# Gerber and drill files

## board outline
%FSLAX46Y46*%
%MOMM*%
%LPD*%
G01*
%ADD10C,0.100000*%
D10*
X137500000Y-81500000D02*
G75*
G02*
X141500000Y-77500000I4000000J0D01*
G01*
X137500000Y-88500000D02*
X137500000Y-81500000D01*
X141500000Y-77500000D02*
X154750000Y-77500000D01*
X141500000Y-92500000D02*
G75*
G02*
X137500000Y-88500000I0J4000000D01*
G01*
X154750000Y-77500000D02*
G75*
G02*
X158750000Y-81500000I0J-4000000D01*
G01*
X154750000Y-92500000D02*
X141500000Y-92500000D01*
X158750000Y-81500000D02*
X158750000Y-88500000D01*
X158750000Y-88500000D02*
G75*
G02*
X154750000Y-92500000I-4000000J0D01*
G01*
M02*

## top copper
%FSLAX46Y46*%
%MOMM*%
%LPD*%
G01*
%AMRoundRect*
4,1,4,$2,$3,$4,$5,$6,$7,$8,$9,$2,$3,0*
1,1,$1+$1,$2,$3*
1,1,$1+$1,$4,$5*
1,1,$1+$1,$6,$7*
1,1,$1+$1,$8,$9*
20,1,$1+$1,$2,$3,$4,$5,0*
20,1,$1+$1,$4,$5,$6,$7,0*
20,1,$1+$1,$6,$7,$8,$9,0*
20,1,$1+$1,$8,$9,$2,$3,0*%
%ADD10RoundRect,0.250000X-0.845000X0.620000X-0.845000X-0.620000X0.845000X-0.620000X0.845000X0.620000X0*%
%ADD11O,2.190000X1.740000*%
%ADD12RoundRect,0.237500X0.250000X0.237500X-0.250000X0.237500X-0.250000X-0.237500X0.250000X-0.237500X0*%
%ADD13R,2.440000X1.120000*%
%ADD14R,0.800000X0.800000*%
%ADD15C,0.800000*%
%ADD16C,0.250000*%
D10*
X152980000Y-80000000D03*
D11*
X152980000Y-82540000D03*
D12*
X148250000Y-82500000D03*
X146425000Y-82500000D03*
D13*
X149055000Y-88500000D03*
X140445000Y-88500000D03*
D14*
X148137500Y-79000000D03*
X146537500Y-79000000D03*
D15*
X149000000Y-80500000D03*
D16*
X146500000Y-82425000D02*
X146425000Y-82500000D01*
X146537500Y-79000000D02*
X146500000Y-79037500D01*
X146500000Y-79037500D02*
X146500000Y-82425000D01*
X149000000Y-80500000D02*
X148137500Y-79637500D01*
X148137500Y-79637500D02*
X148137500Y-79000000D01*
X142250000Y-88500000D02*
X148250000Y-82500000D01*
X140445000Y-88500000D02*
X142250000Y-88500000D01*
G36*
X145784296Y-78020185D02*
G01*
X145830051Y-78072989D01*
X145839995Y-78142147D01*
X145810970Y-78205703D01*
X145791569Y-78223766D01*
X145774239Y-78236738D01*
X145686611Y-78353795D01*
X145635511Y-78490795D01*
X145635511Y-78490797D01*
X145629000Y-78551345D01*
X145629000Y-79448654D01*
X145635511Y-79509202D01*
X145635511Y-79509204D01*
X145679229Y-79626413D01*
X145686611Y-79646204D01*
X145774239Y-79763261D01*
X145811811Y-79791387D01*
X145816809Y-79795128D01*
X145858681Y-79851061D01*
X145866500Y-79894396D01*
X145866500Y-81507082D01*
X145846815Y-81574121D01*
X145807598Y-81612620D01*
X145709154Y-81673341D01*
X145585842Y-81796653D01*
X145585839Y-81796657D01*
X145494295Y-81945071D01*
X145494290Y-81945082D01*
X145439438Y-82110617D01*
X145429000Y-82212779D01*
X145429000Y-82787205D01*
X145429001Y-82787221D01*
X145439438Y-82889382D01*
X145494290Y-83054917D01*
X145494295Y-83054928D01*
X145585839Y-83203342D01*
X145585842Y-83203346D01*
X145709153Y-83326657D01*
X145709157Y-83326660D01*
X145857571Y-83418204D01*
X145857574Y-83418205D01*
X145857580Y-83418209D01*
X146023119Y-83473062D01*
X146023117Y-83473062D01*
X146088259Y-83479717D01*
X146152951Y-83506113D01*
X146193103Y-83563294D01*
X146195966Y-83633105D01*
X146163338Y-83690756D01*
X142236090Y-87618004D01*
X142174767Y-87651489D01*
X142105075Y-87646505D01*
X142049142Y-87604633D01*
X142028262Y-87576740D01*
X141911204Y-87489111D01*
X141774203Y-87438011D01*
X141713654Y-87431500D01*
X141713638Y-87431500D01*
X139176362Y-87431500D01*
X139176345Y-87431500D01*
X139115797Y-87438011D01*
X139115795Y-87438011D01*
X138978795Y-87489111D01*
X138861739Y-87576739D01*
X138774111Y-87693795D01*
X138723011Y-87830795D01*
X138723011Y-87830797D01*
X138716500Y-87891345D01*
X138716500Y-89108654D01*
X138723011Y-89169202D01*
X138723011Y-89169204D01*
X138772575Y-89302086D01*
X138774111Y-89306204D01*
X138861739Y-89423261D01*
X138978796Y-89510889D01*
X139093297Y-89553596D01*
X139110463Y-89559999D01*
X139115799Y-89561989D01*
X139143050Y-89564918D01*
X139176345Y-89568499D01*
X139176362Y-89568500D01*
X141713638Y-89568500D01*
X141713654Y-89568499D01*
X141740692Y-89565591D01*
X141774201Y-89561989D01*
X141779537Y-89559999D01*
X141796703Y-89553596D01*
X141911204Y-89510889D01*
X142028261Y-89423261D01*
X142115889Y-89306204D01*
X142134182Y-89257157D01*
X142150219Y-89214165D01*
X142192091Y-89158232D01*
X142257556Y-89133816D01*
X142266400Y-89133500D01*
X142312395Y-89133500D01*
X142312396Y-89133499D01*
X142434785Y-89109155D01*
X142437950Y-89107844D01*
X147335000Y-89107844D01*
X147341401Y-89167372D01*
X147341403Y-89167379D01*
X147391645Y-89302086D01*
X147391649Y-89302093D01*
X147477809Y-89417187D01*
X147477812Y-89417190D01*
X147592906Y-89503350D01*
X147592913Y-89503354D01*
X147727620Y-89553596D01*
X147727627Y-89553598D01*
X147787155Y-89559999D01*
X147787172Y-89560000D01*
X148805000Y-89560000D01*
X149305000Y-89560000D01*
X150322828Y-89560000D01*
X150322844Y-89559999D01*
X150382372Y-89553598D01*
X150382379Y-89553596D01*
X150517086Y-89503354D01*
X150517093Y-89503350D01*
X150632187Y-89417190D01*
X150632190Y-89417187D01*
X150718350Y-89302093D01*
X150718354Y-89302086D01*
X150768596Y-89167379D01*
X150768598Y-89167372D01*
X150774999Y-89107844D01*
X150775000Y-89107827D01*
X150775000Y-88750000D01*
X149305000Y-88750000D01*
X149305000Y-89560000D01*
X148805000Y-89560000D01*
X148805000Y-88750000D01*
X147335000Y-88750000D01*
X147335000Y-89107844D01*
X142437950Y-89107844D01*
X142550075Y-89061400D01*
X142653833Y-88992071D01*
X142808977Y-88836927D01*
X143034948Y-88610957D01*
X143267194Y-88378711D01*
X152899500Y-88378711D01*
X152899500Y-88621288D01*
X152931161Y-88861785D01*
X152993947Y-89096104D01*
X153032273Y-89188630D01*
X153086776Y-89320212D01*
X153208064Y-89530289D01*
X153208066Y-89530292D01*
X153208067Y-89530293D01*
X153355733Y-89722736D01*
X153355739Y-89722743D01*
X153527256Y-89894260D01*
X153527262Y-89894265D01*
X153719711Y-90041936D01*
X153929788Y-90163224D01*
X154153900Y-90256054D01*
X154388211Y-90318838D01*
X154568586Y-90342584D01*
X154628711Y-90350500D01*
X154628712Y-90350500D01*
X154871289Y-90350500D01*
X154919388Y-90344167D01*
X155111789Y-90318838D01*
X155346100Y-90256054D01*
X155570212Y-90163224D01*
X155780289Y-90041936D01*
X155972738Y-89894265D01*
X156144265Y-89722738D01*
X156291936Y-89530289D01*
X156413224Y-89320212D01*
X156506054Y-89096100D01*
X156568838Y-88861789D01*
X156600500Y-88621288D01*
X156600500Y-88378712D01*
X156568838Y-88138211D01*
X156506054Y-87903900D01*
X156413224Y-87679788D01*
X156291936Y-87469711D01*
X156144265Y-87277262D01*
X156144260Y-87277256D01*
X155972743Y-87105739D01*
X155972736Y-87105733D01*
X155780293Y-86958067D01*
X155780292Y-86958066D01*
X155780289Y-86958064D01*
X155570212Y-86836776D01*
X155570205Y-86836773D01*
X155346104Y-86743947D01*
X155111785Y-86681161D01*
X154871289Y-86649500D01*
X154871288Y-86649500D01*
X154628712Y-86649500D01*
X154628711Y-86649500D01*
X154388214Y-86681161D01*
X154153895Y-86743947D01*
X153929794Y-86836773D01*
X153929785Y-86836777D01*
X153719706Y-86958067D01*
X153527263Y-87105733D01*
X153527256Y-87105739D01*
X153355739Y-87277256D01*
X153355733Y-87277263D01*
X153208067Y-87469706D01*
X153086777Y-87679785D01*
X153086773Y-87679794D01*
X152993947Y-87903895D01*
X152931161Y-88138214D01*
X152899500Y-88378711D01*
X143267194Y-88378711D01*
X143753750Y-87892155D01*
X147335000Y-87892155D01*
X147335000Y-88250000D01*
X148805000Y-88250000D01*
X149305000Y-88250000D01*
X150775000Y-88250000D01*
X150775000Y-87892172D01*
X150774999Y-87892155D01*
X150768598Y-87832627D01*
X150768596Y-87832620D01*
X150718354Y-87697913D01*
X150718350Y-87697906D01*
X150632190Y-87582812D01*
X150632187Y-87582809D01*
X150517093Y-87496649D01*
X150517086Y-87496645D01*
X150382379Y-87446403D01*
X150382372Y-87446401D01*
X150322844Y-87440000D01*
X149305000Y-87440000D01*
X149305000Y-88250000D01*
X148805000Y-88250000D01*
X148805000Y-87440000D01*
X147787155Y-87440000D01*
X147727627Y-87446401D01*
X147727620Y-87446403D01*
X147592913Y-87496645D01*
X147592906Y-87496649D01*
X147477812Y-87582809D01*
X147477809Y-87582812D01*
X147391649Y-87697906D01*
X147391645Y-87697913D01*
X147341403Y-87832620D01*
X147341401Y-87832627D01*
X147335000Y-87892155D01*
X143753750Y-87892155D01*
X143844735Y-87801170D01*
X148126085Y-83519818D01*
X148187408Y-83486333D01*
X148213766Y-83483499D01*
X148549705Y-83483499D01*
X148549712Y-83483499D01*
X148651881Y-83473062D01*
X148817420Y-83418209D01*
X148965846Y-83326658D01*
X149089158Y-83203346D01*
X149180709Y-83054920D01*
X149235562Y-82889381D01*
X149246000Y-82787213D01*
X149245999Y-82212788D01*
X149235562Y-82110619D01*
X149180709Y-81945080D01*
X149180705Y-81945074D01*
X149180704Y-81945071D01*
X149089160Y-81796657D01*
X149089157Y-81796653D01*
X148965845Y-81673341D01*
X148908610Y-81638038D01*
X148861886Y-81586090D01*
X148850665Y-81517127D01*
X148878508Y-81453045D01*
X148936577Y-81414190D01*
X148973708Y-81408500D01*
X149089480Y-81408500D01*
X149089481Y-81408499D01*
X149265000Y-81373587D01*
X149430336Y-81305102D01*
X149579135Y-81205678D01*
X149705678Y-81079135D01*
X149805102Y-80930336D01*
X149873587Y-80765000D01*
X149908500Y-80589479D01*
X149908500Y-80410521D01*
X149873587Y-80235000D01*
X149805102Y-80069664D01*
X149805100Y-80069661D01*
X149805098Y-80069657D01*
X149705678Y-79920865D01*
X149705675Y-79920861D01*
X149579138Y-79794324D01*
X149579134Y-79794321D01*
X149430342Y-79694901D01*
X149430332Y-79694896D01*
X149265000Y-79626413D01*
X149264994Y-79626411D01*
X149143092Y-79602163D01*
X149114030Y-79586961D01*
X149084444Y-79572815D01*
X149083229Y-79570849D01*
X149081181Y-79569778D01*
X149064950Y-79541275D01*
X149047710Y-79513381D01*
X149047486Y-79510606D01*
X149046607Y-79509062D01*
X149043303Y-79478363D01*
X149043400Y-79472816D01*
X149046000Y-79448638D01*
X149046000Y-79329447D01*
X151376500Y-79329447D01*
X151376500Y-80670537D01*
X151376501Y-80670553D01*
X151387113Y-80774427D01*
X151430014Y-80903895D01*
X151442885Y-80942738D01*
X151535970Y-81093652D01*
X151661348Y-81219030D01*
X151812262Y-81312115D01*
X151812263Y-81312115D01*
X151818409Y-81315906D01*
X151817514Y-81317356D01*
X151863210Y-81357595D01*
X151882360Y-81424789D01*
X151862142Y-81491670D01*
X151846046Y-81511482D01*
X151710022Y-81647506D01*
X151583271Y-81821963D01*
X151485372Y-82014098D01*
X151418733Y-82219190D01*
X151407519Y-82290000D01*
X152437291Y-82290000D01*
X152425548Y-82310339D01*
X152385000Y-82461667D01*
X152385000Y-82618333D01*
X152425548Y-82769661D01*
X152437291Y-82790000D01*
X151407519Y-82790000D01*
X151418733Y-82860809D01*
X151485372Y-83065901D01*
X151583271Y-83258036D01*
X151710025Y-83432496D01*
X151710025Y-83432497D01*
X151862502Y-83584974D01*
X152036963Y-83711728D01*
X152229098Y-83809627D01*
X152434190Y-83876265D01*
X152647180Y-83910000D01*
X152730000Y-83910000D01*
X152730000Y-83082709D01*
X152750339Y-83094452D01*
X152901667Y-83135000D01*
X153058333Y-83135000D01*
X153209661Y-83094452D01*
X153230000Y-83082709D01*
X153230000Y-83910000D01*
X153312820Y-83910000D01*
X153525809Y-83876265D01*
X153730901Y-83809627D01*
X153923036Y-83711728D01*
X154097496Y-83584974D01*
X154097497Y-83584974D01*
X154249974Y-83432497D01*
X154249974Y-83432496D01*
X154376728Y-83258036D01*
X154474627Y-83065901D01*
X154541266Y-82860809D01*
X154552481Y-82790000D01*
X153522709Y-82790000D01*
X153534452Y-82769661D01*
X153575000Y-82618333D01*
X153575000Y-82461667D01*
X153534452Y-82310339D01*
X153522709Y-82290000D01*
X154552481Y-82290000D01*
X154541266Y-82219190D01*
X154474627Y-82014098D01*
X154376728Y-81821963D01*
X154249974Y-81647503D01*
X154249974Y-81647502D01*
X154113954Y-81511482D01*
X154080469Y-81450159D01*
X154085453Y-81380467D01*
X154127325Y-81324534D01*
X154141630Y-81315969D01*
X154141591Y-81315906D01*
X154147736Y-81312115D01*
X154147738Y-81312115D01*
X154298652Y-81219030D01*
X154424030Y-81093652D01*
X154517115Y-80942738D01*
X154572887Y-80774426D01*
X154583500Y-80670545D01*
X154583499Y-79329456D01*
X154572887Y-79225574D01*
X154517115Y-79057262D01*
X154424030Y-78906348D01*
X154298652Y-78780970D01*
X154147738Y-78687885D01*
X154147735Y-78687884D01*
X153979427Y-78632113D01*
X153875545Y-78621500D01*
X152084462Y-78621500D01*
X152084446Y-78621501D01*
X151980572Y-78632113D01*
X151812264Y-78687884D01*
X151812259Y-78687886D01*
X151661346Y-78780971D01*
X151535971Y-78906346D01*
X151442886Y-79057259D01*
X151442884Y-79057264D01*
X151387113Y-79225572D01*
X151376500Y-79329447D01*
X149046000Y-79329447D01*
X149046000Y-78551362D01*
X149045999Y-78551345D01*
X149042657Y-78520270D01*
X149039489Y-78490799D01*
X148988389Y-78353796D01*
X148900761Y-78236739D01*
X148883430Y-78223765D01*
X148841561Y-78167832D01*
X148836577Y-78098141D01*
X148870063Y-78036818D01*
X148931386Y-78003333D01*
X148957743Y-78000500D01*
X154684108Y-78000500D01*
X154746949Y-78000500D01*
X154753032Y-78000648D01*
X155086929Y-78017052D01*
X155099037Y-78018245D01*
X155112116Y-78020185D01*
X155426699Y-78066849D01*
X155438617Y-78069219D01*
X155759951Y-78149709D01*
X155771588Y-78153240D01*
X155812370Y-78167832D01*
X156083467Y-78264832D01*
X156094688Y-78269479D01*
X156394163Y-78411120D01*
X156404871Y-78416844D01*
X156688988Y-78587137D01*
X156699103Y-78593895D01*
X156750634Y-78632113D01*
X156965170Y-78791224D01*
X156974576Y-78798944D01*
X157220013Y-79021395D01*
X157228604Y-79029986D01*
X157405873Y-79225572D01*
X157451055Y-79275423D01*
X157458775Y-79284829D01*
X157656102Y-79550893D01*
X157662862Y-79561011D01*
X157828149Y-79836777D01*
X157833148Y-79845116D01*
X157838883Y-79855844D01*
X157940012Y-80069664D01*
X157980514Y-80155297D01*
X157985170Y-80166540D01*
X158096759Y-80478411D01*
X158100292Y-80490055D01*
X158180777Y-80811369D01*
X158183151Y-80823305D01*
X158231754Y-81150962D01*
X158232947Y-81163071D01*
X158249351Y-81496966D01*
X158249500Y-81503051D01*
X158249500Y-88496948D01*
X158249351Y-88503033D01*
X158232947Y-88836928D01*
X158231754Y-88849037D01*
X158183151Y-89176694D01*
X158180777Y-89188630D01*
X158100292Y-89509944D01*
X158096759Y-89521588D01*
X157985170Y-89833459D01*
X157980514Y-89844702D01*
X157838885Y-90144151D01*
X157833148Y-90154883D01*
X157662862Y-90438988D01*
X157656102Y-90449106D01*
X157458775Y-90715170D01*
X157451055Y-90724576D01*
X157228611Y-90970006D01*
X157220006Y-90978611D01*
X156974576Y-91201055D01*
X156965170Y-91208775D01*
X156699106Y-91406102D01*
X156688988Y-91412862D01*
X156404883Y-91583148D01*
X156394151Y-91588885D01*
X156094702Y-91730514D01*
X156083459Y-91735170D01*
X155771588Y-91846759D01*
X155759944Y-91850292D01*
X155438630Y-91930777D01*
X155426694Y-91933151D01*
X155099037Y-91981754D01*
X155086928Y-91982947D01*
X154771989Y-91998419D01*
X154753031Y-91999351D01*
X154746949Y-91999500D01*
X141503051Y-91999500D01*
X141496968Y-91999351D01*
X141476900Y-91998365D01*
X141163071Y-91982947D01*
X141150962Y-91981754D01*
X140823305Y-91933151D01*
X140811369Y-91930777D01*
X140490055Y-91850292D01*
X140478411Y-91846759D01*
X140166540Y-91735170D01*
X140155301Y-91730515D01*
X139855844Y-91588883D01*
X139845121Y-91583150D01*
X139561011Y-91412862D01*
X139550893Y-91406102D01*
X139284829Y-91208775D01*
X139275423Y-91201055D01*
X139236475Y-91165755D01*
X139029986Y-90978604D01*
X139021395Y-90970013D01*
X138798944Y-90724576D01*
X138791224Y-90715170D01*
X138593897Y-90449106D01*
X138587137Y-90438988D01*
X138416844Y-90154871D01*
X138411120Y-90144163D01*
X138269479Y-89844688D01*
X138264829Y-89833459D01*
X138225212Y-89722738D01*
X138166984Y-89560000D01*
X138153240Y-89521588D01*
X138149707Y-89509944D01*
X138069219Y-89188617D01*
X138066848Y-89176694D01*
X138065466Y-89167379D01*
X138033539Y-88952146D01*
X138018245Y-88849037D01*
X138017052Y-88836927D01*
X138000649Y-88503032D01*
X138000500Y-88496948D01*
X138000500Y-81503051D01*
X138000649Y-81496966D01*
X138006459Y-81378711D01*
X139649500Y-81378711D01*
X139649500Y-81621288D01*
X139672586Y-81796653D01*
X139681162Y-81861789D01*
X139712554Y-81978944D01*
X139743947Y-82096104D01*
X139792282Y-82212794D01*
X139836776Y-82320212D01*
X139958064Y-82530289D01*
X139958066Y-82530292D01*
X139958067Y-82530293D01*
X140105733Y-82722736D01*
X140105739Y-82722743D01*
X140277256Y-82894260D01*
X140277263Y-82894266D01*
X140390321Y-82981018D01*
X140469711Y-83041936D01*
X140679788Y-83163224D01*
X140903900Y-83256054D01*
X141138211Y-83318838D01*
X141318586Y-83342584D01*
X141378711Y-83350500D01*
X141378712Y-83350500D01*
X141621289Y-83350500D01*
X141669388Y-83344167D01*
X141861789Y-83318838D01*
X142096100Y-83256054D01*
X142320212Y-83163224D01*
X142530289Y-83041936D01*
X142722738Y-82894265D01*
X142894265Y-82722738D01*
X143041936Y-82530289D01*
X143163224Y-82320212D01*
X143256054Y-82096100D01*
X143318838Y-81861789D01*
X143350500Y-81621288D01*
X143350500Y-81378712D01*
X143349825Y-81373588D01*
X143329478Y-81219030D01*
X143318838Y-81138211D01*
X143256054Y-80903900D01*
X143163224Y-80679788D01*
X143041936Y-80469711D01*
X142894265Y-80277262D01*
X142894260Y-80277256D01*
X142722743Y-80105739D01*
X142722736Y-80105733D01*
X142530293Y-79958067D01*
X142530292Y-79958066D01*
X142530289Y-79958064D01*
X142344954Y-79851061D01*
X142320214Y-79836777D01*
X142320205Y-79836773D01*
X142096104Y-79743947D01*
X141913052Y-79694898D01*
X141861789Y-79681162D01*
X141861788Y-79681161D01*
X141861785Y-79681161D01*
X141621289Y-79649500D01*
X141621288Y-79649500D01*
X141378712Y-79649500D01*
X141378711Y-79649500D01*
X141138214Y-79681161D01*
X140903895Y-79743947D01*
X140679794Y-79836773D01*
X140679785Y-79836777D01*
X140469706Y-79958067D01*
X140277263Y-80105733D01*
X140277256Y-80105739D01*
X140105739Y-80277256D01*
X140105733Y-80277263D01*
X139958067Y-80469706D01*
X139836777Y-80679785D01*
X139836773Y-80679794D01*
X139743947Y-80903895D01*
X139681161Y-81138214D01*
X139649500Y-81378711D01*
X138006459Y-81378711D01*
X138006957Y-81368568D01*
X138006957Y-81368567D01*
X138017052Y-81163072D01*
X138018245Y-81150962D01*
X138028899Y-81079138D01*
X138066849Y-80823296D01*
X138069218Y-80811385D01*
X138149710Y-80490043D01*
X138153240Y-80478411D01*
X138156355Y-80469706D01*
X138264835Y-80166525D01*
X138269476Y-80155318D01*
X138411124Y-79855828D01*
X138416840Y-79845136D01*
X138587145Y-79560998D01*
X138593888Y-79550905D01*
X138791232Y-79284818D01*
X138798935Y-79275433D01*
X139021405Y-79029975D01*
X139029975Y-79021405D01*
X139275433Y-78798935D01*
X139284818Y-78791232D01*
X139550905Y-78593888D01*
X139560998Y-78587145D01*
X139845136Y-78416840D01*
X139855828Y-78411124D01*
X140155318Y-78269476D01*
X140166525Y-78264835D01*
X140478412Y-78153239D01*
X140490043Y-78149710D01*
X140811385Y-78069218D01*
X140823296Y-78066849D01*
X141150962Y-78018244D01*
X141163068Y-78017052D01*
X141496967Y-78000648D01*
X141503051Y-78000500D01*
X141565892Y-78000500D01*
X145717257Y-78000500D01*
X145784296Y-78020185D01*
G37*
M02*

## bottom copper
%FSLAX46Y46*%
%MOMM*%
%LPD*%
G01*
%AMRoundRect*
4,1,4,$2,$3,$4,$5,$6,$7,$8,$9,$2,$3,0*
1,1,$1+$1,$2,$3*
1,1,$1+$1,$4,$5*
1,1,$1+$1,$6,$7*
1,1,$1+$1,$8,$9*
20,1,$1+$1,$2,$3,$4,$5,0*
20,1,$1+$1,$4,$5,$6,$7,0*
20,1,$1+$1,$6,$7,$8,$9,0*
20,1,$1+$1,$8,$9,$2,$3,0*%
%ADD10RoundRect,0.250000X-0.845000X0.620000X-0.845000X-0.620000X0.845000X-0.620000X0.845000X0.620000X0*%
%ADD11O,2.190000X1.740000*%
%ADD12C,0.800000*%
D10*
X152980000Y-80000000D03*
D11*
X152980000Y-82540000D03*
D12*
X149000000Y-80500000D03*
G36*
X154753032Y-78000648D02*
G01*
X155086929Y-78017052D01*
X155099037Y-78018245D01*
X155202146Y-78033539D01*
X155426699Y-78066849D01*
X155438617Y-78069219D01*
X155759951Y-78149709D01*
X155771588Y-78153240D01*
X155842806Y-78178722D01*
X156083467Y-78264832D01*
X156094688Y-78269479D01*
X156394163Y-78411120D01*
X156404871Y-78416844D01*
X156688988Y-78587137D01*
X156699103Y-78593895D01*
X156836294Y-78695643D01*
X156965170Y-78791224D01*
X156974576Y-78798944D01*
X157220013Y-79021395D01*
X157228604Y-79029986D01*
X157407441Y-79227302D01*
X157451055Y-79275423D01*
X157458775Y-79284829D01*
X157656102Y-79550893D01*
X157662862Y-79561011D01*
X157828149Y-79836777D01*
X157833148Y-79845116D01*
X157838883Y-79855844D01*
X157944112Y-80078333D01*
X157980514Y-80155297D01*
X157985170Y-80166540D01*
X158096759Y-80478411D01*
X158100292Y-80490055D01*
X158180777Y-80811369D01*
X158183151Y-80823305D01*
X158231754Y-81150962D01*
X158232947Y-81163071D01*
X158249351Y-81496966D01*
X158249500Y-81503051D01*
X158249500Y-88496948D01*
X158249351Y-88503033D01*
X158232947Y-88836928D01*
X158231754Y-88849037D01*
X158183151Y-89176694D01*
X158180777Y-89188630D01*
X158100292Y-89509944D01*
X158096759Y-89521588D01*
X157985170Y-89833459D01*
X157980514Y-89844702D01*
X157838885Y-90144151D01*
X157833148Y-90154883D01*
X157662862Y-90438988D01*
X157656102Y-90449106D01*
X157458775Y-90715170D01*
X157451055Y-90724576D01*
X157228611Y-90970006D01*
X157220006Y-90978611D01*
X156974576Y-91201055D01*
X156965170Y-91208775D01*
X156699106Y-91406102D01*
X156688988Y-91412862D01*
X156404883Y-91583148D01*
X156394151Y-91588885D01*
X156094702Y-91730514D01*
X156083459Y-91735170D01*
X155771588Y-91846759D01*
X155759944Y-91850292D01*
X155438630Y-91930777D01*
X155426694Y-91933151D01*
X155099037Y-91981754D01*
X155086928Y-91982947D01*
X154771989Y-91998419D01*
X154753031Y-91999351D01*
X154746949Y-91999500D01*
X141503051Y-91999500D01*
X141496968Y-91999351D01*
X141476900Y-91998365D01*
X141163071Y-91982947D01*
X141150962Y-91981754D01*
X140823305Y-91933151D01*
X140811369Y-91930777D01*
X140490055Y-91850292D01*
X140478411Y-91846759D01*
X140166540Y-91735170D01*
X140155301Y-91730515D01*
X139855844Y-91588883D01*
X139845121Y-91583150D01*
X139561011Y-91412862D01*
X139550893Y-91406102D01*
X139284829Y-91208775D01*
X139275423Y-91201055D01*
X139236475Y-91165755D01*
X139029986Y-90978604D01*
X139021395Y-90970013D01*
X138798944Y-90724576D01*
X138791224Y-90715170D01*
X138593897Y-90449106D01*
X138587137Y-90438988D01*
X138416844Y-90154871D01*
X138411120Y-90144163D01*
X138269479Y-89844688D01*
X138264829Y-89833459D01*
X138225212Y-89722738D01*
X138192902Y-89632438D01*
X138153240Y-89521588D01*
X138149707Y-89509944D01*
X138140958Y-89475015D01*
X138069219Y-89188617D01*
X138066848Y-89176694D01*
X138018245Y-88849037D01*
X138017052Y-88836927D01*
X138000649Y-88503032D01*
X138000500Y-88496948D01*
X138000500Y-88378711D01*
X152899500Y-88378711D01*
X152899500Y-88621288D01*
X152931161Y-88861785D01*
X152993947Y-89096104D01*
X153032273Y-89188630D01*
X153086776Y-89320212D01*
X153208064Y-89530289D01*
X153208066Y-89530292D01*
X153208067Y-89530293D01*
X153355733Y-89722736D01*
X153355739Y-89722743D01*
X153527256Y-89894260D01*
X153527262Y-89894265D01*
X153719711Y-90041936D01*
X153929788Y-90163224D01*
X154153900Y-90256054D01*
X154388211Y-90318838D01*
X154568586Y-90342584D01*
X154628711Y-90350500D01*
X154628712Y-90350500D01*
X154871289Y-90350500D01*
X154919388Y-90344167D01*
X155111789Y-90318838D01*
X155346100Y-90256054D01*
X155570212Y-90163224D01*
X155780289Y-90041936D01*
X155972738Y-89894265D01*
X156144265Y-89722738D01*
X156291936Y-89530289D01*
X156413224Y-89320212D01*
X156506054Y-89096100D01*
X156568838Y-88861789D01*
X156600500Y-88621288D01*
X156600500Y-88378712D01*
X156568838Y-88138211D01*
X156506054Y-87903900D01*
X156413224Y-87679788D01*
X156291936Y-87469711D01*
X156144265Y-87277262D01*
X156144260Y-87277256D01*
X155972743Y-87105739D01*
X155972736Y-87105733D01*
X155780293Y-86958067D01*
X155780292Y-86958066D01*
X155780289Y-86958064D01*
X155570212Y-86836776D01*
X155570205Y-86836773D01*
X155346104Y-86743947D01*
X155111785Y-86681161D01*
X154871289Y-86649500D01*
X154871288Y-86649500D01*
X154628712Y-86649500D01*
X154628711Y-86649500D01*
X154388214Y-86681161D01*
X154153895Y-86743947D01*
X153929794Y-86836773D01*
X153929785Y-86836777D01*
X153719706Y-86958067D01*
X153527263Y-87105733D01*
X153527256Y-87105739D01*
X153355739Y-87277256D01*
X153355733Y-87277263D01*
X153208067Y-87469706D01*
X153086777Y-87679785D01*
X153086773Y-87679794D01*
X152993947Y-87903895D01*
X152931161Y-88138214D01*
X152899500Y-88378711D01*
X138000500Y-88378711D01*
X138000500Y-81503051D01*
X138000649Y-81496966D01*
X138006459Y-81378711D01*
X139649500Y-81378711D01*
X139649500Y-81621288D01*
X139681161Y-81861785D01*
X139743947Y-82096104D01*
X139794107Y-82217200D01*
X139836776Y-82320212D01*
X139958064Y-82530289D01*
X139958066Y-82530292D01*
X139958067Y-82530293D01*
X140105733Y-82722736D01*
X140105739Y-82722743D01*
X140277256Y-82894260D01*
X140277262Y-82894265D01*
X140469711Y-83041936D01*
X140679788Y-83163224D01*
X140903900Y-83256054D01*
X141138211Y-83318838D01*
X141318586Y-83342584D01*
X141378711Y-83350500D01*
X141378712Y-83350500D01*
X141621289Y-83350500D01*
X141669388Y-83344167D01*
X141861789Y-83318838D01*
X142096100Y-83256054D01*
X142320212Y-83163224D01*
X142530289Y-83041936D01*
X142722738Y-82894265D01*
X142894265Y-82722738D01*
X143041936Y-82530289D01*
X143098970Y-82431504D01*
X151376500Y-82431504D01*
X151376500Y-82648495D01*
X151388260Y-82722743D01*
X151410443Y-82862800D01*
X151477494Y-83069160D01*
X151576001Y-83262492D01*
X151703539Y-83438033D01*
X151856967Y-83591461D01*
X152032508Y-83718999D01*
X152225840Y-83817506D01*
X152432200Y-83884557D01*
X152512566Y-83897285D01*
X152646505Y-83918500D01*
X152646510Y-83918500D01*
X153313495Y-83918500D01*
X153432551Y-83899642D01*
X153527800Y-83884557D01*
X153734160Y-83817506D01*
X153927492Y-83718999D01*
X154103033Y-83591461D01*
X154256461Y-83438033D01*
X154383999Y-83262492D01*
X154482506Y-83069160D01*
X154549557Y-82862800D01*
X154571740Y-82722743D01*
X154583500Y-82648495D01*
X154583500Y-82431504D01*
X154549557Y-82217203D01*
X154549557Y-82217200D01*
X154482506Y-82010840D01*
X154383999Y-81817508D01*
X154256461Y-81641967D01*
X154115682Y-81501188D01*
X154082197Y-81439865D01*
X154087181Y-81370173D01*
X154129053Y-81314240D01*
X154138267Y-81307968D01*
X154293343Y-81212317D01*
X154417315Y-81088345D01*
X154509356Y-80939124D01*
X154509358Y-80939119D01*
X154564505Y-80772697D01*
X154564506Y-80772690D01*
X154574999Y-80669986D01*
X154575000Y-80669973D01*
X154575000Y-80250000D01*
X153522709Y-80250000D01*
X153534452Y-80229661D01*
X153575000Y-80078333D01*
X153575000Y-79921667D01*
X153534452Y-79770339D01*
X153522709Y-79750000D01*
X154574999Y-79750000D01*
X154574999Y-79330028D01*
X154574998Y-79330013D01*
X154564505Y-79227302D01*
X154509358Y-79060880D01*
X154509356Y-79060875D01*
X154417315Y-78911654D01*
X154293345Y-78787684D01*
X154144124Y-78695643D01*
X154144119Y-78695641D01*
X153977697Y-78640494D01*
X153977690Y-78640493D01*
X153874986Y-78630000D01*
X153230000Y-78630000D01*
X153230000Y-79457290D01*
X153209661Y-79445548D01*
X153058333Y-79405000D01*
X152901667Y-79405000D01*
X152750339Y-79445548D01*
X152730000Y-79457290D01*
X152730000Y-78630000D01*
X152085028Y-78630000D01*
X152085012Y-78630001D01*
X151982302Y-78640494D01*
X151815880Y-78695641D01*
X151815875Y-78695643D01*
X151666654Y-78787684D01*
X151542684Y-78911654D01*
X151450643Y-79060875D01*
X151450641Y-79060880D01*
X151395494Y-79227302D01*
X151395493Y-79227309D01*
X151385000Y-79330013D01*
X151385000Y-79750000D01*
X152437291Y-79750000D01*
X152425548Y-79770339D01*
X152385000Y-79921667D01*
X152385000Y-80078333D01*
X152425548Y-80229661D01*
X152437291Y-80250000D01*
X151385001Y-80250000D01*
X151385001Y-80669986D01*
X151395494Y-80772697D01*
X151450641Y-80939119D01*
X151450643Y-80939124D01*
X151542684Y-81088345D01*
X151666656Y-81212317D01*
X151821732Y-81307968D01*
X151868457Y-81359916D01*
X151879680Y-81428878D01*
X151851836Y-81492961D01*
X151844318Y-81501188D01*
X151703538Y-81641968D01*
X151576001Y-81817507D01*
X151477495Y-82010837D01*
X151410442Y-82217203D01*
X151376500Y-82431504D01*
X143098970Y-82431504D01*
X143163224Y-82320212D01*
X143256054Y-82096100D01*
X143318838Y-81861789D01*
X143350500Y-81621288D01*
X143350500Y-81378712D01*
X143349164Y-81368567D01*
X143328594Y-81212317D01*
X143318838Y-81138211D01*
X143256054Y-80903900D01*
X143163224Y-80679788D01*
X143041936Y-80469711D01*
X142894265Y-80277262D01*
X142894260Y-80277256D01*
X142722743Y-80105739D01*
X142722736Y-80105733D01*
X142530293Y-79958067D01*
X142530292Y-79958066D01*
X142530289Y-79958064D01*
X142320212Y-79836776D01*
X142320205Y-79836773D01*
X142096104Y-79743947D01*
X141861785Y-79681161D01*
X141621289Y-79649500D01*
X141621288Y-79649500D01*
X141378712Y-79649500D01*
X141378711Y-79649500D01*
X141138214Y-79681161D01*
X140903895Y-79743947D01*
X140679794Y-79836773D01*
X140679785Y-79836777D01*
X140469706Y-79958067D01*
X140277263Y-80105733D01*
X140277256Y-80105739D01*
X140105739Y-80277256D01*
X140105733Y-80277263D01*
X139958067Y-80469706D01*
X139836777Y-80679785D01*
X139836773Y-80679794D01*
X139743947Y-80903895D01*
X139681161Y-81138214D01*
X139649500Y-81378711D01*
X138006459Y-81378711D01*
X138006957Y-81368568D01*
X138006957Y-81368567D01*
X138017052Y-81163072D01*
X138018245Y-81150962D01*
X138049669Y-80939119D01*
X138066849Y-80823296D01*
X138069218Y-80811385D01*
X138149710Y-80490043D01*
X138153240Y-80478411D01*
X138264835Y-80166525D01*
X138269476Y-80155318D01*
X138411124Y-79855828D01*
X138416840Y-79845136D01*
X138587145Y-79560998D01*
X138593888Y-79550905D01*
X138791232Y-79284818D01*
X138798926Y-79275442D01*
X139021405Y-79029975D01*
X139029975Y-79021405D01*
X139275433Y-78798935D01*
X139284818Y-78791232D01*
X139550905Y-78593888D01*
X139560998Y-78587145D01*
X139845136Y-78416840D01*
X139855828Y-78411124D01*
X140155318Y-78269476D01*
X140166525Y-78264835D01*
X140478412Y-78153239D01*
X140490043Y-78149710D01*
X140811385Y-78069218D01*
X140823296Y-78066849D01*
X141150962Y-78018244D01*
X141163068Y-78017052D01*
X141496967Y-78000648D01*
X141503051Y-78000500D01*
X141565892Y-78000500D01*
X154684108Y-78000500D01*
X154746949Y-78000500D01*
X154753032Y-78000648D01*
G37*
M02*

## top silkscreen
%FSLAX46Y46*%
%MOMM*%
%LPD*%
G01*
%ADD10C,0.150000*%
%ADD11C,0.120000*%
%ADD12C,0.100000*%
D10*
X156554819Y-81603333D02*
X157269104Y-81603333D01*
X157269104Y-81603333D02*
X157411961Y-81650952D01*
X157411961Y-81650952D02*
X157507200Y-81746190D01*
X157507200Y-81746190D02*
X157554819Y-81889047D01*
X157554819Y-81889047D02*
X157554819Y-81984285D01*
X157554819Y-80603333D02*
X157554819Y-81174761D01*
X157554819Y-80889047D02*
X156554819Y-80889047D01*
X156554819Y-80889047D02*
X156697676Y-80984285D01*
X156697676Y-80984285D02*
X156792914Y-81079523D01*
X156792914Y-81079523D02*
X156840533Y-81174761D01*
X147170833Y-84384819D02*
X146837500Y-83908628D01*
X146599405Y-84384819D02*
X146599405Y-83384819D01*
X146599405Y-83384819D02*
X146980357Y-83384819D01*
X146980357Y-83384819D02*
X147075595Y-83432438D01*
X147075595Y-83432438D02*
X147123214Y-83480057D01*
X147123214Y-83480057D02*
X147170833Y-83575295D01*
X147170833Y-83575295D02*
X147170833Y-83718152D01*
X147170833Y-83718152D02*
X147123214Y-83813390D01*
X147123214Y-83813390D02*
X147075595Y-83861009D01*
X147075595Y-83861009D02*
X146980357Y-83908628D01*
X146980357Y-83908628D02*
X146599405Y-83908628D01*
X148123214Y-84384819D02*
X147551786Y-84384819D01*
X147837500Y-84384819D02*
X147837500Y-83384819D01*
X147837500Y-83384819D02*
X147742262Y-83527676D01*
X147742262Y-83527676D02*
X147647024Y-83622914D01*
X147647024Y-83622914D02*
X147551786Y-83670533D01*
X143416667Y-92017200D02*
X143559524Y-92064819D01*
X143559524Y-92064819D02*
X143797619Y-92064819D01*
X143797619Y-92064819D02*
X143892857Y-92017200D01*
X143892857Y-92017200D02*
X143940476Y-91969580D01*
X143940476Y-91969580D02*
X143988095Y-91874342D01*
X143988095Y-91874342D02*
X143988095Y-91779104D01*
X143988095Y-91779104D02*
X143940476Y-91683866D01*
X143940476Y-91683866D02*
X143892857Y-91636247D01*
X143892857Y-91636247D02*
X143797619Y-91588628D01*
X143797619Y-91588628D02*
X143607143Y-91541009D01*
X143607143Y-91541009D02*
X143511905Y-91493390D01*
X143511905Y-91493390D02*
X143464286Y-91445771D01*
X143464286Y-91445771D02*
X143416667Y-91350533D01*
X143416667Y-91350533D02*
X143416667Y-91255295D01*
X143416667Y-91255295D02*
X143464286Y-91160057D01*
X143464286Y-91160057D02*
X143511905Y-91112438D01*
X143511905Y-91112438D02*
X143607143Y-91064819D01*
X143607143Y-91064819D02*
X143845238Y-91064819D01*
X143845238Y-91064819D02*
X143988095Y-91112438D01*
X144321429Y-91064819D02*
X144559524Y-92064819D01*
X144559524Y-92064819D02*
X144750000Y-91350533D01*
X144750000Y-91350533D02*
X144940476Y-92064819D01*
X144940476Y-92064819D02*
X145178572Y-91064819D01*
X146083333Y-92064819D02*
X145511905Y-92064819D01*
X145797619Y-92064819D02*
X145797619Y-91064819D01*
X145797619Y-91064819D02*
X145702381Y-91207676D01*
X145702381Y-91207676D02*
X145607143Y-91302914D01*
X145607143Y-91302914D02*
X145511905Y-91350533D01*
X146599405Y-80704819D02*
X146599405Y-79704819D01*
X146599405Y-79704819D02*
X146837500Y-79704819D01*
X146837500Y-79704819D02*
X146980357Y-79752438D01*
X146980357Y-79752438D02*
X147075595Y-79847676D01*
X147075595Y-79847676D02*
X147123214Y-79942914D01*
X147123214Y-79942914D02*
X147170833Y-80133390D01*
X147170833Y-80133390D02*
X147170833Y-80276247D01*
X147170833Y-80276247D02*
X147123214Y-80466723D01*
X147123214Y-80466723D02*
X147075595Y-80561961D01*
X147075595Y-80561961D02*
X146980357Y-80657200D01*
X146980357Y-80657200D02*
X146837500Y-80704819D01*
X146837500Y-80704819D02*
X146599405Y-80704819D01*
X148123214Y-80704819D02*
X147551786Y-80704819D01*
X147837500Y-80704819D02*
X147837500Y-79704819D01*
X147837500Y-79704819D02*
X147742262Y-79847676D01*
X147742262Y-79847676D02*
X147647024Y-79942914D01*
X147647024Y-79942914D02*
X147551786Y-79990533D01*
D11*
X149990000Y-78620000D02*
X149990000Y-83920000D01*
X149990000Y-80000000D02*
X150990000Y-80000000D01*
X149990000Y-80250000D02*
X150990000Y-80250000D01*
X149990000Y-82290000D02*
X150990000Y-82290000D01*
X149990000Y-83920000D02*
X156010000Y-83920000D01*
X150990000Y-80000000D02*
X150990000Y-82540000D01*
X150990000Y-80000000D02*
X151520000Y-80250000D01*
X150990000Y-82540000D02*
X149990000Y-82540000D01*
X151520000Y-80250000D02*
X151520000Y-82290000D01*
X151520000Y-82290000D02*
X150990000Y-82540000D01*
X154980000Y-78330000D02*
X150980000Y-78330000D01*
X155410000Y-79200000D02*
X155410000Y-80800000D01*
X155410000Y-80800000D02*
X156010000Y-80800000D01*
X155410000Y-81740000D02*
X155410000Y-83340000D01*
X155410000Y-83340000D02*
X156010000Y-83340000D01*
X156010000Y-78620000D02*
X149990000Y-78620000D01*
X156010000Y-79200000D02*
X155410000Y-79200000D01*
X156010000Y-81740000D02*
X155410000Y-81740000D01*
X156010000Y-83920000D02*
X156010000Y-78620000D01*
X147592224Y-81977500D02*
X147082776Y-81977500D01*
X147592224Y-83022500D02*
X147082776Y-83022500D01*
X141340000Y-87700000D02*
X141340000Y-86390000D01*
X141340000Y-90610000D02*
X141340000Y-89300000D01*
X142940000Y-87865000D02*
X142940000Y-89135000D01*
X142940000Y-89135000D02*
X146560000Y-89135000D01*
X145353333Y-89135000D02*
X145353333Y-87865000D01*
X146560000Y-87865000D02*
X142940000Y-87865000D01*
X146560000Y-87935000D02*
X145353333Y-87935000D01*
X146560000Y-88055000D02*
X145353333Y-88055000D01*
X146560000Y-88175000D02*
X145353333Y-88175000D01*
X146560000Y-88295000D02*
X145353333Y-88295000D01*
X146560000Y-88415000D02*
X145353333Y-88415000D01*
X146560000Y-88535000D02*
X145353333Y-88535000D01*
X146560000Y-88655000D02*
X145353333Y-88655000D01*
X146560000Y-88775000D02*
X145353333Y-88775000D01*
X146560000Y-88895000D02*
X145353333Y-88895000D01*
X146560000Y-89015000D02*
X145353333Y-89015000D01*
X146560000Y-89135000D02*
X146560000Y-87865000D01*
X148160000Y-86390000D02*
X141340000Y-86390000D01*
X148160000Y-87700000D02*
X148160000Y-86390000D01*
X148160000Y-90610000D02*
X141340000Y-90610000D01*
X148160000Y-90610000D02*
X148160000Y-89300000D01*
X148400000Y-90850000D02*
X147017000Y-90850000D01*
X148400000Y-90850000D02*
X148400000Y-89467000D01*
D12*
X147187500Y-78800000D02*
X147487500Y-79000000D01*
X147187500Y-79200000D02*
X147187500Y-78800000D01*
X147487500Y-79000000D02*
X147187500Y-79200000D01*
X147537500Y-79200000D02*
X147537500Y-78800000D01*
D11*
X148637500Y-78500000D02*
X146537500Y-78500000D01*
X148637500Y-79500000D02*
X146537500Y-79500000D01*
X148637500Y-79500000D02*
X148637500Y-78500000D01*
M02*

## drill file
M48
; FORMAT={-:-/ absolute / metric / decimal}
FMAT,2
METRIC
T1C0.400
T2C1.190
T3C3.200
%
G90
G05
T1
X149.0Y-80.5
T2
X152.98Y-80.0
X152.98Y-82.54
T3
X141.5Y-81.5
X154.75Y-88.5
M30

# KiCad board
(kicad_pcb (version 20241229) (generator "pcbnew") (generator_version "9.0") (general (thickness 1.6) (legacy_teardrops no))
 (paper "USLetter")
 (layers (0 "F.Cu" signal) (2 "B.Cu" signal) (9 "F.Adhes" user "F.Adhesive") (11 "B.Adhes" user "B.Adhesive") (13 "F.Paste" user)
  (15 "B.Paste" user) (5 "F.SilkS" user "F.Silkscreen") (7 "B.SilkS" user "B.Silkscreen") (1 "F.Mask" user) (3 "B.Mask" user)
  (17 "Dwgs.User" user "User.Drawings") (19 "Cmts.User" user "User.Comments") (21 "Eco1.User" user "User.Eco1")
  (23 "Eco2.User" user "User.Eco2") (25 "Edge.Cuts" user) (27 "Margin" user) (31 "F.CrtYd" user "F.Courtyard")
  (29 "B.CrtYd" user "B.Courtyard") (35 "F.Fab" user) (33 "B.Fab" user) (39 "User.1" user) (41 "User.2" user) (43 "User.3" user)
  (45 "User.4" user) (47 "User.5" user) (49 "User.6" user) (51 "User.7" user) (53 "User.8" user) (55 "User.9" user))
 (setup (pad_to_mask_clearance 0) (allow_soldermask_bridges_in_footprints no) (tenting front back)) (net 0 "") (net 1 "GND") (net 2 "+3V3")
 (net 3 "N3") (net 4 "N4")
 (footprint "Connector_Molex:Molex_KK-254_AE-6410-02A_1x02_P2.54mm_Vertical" (layer "F.Cu") (at 152.98 80 -90)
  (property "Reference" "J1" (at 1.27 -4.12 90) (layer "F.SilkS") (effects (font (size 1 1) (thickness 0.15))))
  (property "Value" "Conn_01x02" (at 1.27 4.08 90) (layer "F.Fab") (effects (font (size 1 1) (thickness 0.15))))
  (fp_line (start -1.38 2.99) (end 3.92 2.99) (stroke (width 0.12) (type solid)) (layer "F.SilkS"))
  (fp_line (start 0 2.99) (end 0 1.99) (stroke (width 0.12) (type solid)) (layer "F.SilkS"))
  (fp_line (start 0.25 2.99) (end 0.25 1.99) (stroke (width 0.12) (type solid)) (layer "F.SilkS"))
  (fp_line (start 2.29 2.99) (end 2.29 1.99) (stroke (width 0.12) (type solid)) (layer "F.SilkS"))
  (fp_line (start 3.92 2.99) (end 3.92 -3.03) (stroke (width 0.12) (type solid)) (layer "F.SilkS"))
  (fp_line (start 0 1.99) (end 2.54 1.99) (stroke (width 0.12) (type solid)) (layer "F.SilkS"))
  (fp_line (start 0 1.99) (end 0.25 1.46) (stroke (width 0.12) (type solid)) (layer "F.SilkS"))
  (fp_line (start 2.54 1.99) (end 2.54 2.99) (stroke (width 0.12) (type solid)) (layer "F.SilkS"))
  (fp_line (start 0.25 1.46) (end 2.29 1.46) (stroke (width 0.12) (type solid)) (layer "F.SilkS"))
  (fp_line (start 2.29 1.46) (end 2.54 1.99) (stroke (width 0.12) (type solid)) (layer "F.SilkS"))
  (fp_line (start -1.67 -2) (end -1.67 2) (stroke (width 0.12) (type solid)) (layer "F.SilkS"))
  (fp_line (start -0.8 -2.43) (end 0.8 -2.43) (stroke (width 0.12) (type solid)) (layer "F.SilkS"))
  (fp_line (start 0.8 -2.43) (end 0.8 -3.03) (stroke (width 0.12) (type solid)) (layer "F.SilkS"))
  (fp_line (start 1.74 -2.43) (end 3.34 -2.43) (stroke (width 0.12) (type solid)) (layer "F.SilkS"))
  (fp_line (start 3.34 -2.43) (end 3.34 -3.03) (stroke (width 0.12) (type solid)) (layer "F.SilkS"))
  (fp_line (start -1.38 -3.03) (end -1.38 2.99) (stroke (width 0.12) (type solid)) (layer "F.SilkS"))
  (fp_line (start -0.8 -3.03) (end -0.8 -2.43) (stroke (width 0.12) (type solid)) (layer "F.SilkS"))
  (fp_line (start 1.74 -3.03) (end 1.74 -2.43) (stroke (width 0.12) (type solid)) (layer "F.SilkS"))
  (fp_line (start 3.92 -3.03) (end -1.38 -3.03) (stroke (width 0.12) (type solid)) (layer "F.SilkS"))
  (pad "1" thru_hole roundrect (at 0 0 270) (size 1.74 2.19) (drill 1.19) (layers "*.Cu" "*.Mask") (remove_unused_layers no)
   (roundrect_rratio 0.143678) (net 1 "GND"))
  (pad "2" thru_hole oval (at 2.54 0 270) (size 1.74 2.19) (drill 1.19) (layers "*.Cu" "*.Mask") (remove_unused_layers no) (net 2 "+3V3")))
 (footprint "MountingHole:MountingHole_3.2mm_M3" (layer "F.Cu") (at 141.5 81.5)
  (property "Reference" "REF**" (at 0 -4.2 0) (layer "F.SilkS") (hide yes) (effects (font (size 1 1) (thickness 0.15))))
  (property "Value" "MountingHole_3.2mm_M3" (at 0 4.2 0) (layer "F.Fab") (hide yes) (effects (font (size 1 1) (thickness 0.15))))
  (pad "" np_thru_hole circle (at 0 0) (size 3.2 3.2) (drill 3.2) (layers "*.Cu" "*.Mask")))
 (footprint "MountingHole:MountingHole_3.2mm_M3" (layer "F.Cu") (at 154.75 88.5)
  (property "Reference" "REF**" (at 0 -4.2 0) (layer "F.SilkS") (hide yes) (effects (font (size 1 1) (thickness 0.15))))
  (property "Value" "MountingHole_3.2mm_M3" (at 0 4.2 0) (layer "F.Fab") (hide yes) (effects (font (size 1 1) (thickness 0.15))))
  (pad "" np_thru_hole circle (at 0 0) (size 3.2 3.2) (drill 3.2) (layers "*.Cu" "*.Mask")))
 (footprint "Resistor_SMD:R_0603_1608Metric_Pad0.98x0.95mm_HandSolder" (layer "F.Cu") (at 147.3375 82.5 180)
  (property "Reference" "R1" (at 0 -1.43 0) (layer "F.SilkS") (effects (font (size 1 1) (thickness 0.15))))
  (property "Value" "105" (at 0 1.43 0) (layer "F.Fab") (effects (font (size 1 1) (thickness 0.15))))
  (fp_line (start -0.254724 0.5225) (end 0.254724 0.5225) (stroke (width 0.12) (type solid)) (layer "F.SilkS"))
  (fp_line (start -0.254724 -0.5225) (end 0.254724 -0.5225) (stroke (width 0.12) (type solid)) (layer "F.SilkS"))
  (pad "1" smd roundrect (at -0.9125 0 180) (size 0.975 0.95) (layers "F.Cu" "F.Mask" "F.Paste") (roundrect_rratio 0.25) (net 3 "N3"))
  (pad "2" smd roundrect (at 0.9125 0 180) (size 0.975 0.95) (layers "F.Cu" "F.Mask" "F.Paste") (roundrect_rratio 0.25) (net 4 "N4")))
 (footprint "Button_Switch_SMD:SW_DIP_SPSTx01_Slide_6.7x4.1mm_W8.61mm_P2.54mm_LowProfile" (layer "F.Cu") (at 144.75 88.5 180)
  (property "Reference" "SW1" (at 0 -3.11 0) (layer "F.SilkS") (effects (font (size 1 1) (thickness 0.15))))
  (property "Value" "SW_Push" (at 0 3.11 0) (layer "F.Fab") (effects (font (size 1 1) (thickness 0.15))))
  (fp_line (start 3.41 0.8) (end 3.41 2.11) (stroke (width 0.12) (type solid)) (layer "F.SilkS"))
  (fp_line (start 3.41 -2.11) (end 3.41 -0.8) (stroke (width 0.12) (type solid)) (layer "F.SilkS"))
  (fp_line (start 1.81 0.635) (end 1.81 -0.635) (stroke (width 0.12) (type solid)) (layer "F.SilkS"))
  (fp_line (start 1.81 -0.635) (end -1.81 -0.635) (stroke (width 0.12) (type solid)) (layer "F.SilkS"))
  (fp_line (start -0.603333 -0.635) (end -0.603333 0.635) (stroke (width 0.12) (type solid)) (layer "F.SilkS"))
  (fp_line (start -1.81 0.635) (end 1.81 0.635) (stroke (width 0.12) (type solid)) (layer "F.SilkS"))
  (fp_line (start -1.81 0.565) (end -0.603333 0.565) (stroke (width 0.12) (type solid)) (layer "F.SilkS"))
  (fp_line (start -1.81 0.445) (end -0.603333 0.445) (stroke (width 0.12) (type solid)) (layer "F.SilkS"))
  (fp_line (start -1.81 0.325) (end -0.603333 0.325) (stroke (width 0.12) (type solid)) (layer "F.SilkS"))
  (fp_line (start -1.81 0.205) (end -0.603333 0.205) (stroke (width 0.12) (type solid)) (layer "F.SilkS"))
  (fp_line (start -1.81 0.085) (end -0.603333 0.085) (stroke (width 0.12) (type solid)) (layer "F.SilkS"))
  (fp_line (start -1.81 -0.035) (end -0.603333 -0.035) (stroke (width 0.12) (type solid)) (layer "F.SilkS"))
  (fp_line (start -1.81 -0.155) (end -0.603333 -0.155) (stroke (width 0.12) (type solid)) (layer "F.SilkS"))
  (fp_line (start -1.81 -0.275) (end -0.603333 -0.275) (stroke (width 0.12) (type solid)) (layer "F.SilkS"))
  (fp_line (start -1.81 -0.395) (end -0.603333 -0.395) (stroke (width 0.12) (type solid)) (layer "F.SilkS"))
  (fp_line (start -1.81 -0.515) (end -0.603333 -0.515) (stroke (width 0.12) (type solid)) (layer "F.SilkS"))
  (fp_line (start -1.81 -0.635) (end -1.81 0.635) (stroke (width 0.12) (type solid)) (layer "F.SilkS"))
  (fp_line (start -3.41 2.11) (end 3.41 2.11) (stroke (width 0.12) (type solid)) (layer "F.SilkS"))
  (fp_line (start -3.41 0.8) (end -3.41 2.11) (stroke (width 0.12) (type solid)) (layer "F.SilkS"))
  (fp_line (start -3.41 -2.11) (end 3.41 -2.11) (stroke (width 0.12) (type solid)) (layer "F.SilkS"))
  (fp_line (start -3.41 -2.11) (end -3.41 -0.8) (stroke (width 0.12) (type solid)) (layer "F.SilkS"))
  (fp_line (start -3.65 -2.35) (end -2.267 -2.35) (stroke (width 0.12) (type solid)) (layer "F.SilkS"))
  (fp_line (start -3.65 -2.35) (end -3.65 -0.967) (stroke (width 0.12) (type solid)) (layer "F.SilkS"))
  (pad "1" smd rect (at -4.305 0 180) (size 2.44 1.12) (layers "F.Cu" "F.Mask" "F.Paste") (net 2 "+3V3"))
  (pad "2" smd rect (at 4.305 0 180) (size 2.44 1.12) (layers "F.Cu" "F.Mask" "F.Paste") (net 3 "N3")))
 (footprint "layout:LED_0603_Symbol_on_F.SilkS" (layer "F.Cu") (at 147.3375 79 180)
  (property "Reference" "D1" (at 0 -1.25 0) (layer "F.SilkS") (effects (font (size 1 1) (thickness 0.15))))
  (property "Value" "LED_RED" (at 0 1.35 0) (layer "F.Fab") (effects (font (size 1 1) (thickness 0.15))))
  (fp_line (start 0.15 0.2) (end -0.15 0) (stroke (width 0.1) (type solid)) (layer "F.SilkS"))
  (fp_line (start 0.15 -0.2) (end 0.15 0.2) (stroke (width 0.1) (type solid)) (layer "F.SilkS"))
  (fp_line (start -0.15 0) (end 0.15 -0.2) (stroke (width 0.1) (type solid)) (layer "F.SilkS"))
  (fp_line (start -0.2 -0.2) (end -0.2 0.2) (stroke (width 0.1) (type solid)) (layer "F.SilkS"))
  (fp_line (start -1.3 0.5) (end 0.8 0.5) (stroke (width 0.12) (type solid)) (layer "F.SilkS"))
  (fp_line (start -1.3 -0.5) (end 0.8 -0.5) (stroke (width 0.12) (type solid)) (layer "F.SilkS"))
  (fp_line (start -1.3 -0.5) (end -1.3 0.5) (stroke (width 0.12) (type solid)) (layer "F.SilkS"))
  (pad "1" smd rect (at -0.8 0) (size 0.8 0.8) (layers "F.Cu" "F.Mask" "F.Paste") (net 1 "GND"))
  (pad "2" smd rect (at 0.8 0) (size 0.8 0.8) (layers "F.Cu" "F.Mask" "F.Paste") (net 4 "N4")))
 (gr_arc (start 137.5 81.5) (mid 138.671573 78.671573) (end 141.5 77.5) (stroke (width 0.1) (type default)) (layer "Edge.Cuts"))
 (gr_line (start 137.5 88.5) (end 137.5 81.5) (stroke (width 0.1) (type default)) (layer "Edge.Cuts"))
 (gr_line (start 141.5 77.5) (end 154.75 77.5) (stroke (width 0.1) (type default)) (layer "Edge.Cuts"))
 (gr_arc (start 141.5 92.5) (mid 138.671573 91.328427) (end 137.5 88.5) (stroke (width 0.1) (type default)) (layer "Edge.Cuts"))
 (gr_arc (start 154.75 77.5) (mid 157.578427 78.671573) (end 158.75 81.5) (stroke (width 0.1) (type default)) (layer "Edge.Cuts"))
 (gr_line (start 154.75 92.5) (end 141.5 92.5) (stroke (width 0.1) (type default)) (layer "Edge.Cuts"))
 (gr_line (start 158.75 81.5) (end 158.75 88.5) (stroke (width 0.1) (type default)) (layer "Edge.Cuts"))
 (gr_arc (start 158.75 88.5) (mid 157.578427 91.328427) (end 154.75 92.5) (stroke (width 0.1) (type default)) (layer "Edge.Cuts"))
 (segment (start 146.5 82.425) (end 146.425 82.5) (width 0.25) (layer "F.Cu") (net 4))
 (segment (start 146.5375 79) (end 146.5 79.0375) (width 0.25) (layer "F.Cu") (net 4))
 (segment (start 146.5 79.0375) (end 146.5 82.425) (width 0.25) (layer "F.Cu") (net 4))
 (segment (start 149 80.5) (end 148.1375 79.6375) (width 0.25) (layer "F.Cu") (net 1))
 (segment (start 148.1375 79.6375) (end 148.1375 79) (width 0.25) (layer "F.Cu") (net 1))
 (via (at 149 80.5) (size 0.8) (drill 0.4) (layers "F.Cu" "B.Cu") (free yes) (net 1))
 (segment (start 142.25 88.5) (end 148.25 82.5) (width 0.25) (layer "F.Cu") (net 3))
 (segment (start 140.445 88.5) (end 142.25 88.5) (width 0.25) (layer "F.Cu") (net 3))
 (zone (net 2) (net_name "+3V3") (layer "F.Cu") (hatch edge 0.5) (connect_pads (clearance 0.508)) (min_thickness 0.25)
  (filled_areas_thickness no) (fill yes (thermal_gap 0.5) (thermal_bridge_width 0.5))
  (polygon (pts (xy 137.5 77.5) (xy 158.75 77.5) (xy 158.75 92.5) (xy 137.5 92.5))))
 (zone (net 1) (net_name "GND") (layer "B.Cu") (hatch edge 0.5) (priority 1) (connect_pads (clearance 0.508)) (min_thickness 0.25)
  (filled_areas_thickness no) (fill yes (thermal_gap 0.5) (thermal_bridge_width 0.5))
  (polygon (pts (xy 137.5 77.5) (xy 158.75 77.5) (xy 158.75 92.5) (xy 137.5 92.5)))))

